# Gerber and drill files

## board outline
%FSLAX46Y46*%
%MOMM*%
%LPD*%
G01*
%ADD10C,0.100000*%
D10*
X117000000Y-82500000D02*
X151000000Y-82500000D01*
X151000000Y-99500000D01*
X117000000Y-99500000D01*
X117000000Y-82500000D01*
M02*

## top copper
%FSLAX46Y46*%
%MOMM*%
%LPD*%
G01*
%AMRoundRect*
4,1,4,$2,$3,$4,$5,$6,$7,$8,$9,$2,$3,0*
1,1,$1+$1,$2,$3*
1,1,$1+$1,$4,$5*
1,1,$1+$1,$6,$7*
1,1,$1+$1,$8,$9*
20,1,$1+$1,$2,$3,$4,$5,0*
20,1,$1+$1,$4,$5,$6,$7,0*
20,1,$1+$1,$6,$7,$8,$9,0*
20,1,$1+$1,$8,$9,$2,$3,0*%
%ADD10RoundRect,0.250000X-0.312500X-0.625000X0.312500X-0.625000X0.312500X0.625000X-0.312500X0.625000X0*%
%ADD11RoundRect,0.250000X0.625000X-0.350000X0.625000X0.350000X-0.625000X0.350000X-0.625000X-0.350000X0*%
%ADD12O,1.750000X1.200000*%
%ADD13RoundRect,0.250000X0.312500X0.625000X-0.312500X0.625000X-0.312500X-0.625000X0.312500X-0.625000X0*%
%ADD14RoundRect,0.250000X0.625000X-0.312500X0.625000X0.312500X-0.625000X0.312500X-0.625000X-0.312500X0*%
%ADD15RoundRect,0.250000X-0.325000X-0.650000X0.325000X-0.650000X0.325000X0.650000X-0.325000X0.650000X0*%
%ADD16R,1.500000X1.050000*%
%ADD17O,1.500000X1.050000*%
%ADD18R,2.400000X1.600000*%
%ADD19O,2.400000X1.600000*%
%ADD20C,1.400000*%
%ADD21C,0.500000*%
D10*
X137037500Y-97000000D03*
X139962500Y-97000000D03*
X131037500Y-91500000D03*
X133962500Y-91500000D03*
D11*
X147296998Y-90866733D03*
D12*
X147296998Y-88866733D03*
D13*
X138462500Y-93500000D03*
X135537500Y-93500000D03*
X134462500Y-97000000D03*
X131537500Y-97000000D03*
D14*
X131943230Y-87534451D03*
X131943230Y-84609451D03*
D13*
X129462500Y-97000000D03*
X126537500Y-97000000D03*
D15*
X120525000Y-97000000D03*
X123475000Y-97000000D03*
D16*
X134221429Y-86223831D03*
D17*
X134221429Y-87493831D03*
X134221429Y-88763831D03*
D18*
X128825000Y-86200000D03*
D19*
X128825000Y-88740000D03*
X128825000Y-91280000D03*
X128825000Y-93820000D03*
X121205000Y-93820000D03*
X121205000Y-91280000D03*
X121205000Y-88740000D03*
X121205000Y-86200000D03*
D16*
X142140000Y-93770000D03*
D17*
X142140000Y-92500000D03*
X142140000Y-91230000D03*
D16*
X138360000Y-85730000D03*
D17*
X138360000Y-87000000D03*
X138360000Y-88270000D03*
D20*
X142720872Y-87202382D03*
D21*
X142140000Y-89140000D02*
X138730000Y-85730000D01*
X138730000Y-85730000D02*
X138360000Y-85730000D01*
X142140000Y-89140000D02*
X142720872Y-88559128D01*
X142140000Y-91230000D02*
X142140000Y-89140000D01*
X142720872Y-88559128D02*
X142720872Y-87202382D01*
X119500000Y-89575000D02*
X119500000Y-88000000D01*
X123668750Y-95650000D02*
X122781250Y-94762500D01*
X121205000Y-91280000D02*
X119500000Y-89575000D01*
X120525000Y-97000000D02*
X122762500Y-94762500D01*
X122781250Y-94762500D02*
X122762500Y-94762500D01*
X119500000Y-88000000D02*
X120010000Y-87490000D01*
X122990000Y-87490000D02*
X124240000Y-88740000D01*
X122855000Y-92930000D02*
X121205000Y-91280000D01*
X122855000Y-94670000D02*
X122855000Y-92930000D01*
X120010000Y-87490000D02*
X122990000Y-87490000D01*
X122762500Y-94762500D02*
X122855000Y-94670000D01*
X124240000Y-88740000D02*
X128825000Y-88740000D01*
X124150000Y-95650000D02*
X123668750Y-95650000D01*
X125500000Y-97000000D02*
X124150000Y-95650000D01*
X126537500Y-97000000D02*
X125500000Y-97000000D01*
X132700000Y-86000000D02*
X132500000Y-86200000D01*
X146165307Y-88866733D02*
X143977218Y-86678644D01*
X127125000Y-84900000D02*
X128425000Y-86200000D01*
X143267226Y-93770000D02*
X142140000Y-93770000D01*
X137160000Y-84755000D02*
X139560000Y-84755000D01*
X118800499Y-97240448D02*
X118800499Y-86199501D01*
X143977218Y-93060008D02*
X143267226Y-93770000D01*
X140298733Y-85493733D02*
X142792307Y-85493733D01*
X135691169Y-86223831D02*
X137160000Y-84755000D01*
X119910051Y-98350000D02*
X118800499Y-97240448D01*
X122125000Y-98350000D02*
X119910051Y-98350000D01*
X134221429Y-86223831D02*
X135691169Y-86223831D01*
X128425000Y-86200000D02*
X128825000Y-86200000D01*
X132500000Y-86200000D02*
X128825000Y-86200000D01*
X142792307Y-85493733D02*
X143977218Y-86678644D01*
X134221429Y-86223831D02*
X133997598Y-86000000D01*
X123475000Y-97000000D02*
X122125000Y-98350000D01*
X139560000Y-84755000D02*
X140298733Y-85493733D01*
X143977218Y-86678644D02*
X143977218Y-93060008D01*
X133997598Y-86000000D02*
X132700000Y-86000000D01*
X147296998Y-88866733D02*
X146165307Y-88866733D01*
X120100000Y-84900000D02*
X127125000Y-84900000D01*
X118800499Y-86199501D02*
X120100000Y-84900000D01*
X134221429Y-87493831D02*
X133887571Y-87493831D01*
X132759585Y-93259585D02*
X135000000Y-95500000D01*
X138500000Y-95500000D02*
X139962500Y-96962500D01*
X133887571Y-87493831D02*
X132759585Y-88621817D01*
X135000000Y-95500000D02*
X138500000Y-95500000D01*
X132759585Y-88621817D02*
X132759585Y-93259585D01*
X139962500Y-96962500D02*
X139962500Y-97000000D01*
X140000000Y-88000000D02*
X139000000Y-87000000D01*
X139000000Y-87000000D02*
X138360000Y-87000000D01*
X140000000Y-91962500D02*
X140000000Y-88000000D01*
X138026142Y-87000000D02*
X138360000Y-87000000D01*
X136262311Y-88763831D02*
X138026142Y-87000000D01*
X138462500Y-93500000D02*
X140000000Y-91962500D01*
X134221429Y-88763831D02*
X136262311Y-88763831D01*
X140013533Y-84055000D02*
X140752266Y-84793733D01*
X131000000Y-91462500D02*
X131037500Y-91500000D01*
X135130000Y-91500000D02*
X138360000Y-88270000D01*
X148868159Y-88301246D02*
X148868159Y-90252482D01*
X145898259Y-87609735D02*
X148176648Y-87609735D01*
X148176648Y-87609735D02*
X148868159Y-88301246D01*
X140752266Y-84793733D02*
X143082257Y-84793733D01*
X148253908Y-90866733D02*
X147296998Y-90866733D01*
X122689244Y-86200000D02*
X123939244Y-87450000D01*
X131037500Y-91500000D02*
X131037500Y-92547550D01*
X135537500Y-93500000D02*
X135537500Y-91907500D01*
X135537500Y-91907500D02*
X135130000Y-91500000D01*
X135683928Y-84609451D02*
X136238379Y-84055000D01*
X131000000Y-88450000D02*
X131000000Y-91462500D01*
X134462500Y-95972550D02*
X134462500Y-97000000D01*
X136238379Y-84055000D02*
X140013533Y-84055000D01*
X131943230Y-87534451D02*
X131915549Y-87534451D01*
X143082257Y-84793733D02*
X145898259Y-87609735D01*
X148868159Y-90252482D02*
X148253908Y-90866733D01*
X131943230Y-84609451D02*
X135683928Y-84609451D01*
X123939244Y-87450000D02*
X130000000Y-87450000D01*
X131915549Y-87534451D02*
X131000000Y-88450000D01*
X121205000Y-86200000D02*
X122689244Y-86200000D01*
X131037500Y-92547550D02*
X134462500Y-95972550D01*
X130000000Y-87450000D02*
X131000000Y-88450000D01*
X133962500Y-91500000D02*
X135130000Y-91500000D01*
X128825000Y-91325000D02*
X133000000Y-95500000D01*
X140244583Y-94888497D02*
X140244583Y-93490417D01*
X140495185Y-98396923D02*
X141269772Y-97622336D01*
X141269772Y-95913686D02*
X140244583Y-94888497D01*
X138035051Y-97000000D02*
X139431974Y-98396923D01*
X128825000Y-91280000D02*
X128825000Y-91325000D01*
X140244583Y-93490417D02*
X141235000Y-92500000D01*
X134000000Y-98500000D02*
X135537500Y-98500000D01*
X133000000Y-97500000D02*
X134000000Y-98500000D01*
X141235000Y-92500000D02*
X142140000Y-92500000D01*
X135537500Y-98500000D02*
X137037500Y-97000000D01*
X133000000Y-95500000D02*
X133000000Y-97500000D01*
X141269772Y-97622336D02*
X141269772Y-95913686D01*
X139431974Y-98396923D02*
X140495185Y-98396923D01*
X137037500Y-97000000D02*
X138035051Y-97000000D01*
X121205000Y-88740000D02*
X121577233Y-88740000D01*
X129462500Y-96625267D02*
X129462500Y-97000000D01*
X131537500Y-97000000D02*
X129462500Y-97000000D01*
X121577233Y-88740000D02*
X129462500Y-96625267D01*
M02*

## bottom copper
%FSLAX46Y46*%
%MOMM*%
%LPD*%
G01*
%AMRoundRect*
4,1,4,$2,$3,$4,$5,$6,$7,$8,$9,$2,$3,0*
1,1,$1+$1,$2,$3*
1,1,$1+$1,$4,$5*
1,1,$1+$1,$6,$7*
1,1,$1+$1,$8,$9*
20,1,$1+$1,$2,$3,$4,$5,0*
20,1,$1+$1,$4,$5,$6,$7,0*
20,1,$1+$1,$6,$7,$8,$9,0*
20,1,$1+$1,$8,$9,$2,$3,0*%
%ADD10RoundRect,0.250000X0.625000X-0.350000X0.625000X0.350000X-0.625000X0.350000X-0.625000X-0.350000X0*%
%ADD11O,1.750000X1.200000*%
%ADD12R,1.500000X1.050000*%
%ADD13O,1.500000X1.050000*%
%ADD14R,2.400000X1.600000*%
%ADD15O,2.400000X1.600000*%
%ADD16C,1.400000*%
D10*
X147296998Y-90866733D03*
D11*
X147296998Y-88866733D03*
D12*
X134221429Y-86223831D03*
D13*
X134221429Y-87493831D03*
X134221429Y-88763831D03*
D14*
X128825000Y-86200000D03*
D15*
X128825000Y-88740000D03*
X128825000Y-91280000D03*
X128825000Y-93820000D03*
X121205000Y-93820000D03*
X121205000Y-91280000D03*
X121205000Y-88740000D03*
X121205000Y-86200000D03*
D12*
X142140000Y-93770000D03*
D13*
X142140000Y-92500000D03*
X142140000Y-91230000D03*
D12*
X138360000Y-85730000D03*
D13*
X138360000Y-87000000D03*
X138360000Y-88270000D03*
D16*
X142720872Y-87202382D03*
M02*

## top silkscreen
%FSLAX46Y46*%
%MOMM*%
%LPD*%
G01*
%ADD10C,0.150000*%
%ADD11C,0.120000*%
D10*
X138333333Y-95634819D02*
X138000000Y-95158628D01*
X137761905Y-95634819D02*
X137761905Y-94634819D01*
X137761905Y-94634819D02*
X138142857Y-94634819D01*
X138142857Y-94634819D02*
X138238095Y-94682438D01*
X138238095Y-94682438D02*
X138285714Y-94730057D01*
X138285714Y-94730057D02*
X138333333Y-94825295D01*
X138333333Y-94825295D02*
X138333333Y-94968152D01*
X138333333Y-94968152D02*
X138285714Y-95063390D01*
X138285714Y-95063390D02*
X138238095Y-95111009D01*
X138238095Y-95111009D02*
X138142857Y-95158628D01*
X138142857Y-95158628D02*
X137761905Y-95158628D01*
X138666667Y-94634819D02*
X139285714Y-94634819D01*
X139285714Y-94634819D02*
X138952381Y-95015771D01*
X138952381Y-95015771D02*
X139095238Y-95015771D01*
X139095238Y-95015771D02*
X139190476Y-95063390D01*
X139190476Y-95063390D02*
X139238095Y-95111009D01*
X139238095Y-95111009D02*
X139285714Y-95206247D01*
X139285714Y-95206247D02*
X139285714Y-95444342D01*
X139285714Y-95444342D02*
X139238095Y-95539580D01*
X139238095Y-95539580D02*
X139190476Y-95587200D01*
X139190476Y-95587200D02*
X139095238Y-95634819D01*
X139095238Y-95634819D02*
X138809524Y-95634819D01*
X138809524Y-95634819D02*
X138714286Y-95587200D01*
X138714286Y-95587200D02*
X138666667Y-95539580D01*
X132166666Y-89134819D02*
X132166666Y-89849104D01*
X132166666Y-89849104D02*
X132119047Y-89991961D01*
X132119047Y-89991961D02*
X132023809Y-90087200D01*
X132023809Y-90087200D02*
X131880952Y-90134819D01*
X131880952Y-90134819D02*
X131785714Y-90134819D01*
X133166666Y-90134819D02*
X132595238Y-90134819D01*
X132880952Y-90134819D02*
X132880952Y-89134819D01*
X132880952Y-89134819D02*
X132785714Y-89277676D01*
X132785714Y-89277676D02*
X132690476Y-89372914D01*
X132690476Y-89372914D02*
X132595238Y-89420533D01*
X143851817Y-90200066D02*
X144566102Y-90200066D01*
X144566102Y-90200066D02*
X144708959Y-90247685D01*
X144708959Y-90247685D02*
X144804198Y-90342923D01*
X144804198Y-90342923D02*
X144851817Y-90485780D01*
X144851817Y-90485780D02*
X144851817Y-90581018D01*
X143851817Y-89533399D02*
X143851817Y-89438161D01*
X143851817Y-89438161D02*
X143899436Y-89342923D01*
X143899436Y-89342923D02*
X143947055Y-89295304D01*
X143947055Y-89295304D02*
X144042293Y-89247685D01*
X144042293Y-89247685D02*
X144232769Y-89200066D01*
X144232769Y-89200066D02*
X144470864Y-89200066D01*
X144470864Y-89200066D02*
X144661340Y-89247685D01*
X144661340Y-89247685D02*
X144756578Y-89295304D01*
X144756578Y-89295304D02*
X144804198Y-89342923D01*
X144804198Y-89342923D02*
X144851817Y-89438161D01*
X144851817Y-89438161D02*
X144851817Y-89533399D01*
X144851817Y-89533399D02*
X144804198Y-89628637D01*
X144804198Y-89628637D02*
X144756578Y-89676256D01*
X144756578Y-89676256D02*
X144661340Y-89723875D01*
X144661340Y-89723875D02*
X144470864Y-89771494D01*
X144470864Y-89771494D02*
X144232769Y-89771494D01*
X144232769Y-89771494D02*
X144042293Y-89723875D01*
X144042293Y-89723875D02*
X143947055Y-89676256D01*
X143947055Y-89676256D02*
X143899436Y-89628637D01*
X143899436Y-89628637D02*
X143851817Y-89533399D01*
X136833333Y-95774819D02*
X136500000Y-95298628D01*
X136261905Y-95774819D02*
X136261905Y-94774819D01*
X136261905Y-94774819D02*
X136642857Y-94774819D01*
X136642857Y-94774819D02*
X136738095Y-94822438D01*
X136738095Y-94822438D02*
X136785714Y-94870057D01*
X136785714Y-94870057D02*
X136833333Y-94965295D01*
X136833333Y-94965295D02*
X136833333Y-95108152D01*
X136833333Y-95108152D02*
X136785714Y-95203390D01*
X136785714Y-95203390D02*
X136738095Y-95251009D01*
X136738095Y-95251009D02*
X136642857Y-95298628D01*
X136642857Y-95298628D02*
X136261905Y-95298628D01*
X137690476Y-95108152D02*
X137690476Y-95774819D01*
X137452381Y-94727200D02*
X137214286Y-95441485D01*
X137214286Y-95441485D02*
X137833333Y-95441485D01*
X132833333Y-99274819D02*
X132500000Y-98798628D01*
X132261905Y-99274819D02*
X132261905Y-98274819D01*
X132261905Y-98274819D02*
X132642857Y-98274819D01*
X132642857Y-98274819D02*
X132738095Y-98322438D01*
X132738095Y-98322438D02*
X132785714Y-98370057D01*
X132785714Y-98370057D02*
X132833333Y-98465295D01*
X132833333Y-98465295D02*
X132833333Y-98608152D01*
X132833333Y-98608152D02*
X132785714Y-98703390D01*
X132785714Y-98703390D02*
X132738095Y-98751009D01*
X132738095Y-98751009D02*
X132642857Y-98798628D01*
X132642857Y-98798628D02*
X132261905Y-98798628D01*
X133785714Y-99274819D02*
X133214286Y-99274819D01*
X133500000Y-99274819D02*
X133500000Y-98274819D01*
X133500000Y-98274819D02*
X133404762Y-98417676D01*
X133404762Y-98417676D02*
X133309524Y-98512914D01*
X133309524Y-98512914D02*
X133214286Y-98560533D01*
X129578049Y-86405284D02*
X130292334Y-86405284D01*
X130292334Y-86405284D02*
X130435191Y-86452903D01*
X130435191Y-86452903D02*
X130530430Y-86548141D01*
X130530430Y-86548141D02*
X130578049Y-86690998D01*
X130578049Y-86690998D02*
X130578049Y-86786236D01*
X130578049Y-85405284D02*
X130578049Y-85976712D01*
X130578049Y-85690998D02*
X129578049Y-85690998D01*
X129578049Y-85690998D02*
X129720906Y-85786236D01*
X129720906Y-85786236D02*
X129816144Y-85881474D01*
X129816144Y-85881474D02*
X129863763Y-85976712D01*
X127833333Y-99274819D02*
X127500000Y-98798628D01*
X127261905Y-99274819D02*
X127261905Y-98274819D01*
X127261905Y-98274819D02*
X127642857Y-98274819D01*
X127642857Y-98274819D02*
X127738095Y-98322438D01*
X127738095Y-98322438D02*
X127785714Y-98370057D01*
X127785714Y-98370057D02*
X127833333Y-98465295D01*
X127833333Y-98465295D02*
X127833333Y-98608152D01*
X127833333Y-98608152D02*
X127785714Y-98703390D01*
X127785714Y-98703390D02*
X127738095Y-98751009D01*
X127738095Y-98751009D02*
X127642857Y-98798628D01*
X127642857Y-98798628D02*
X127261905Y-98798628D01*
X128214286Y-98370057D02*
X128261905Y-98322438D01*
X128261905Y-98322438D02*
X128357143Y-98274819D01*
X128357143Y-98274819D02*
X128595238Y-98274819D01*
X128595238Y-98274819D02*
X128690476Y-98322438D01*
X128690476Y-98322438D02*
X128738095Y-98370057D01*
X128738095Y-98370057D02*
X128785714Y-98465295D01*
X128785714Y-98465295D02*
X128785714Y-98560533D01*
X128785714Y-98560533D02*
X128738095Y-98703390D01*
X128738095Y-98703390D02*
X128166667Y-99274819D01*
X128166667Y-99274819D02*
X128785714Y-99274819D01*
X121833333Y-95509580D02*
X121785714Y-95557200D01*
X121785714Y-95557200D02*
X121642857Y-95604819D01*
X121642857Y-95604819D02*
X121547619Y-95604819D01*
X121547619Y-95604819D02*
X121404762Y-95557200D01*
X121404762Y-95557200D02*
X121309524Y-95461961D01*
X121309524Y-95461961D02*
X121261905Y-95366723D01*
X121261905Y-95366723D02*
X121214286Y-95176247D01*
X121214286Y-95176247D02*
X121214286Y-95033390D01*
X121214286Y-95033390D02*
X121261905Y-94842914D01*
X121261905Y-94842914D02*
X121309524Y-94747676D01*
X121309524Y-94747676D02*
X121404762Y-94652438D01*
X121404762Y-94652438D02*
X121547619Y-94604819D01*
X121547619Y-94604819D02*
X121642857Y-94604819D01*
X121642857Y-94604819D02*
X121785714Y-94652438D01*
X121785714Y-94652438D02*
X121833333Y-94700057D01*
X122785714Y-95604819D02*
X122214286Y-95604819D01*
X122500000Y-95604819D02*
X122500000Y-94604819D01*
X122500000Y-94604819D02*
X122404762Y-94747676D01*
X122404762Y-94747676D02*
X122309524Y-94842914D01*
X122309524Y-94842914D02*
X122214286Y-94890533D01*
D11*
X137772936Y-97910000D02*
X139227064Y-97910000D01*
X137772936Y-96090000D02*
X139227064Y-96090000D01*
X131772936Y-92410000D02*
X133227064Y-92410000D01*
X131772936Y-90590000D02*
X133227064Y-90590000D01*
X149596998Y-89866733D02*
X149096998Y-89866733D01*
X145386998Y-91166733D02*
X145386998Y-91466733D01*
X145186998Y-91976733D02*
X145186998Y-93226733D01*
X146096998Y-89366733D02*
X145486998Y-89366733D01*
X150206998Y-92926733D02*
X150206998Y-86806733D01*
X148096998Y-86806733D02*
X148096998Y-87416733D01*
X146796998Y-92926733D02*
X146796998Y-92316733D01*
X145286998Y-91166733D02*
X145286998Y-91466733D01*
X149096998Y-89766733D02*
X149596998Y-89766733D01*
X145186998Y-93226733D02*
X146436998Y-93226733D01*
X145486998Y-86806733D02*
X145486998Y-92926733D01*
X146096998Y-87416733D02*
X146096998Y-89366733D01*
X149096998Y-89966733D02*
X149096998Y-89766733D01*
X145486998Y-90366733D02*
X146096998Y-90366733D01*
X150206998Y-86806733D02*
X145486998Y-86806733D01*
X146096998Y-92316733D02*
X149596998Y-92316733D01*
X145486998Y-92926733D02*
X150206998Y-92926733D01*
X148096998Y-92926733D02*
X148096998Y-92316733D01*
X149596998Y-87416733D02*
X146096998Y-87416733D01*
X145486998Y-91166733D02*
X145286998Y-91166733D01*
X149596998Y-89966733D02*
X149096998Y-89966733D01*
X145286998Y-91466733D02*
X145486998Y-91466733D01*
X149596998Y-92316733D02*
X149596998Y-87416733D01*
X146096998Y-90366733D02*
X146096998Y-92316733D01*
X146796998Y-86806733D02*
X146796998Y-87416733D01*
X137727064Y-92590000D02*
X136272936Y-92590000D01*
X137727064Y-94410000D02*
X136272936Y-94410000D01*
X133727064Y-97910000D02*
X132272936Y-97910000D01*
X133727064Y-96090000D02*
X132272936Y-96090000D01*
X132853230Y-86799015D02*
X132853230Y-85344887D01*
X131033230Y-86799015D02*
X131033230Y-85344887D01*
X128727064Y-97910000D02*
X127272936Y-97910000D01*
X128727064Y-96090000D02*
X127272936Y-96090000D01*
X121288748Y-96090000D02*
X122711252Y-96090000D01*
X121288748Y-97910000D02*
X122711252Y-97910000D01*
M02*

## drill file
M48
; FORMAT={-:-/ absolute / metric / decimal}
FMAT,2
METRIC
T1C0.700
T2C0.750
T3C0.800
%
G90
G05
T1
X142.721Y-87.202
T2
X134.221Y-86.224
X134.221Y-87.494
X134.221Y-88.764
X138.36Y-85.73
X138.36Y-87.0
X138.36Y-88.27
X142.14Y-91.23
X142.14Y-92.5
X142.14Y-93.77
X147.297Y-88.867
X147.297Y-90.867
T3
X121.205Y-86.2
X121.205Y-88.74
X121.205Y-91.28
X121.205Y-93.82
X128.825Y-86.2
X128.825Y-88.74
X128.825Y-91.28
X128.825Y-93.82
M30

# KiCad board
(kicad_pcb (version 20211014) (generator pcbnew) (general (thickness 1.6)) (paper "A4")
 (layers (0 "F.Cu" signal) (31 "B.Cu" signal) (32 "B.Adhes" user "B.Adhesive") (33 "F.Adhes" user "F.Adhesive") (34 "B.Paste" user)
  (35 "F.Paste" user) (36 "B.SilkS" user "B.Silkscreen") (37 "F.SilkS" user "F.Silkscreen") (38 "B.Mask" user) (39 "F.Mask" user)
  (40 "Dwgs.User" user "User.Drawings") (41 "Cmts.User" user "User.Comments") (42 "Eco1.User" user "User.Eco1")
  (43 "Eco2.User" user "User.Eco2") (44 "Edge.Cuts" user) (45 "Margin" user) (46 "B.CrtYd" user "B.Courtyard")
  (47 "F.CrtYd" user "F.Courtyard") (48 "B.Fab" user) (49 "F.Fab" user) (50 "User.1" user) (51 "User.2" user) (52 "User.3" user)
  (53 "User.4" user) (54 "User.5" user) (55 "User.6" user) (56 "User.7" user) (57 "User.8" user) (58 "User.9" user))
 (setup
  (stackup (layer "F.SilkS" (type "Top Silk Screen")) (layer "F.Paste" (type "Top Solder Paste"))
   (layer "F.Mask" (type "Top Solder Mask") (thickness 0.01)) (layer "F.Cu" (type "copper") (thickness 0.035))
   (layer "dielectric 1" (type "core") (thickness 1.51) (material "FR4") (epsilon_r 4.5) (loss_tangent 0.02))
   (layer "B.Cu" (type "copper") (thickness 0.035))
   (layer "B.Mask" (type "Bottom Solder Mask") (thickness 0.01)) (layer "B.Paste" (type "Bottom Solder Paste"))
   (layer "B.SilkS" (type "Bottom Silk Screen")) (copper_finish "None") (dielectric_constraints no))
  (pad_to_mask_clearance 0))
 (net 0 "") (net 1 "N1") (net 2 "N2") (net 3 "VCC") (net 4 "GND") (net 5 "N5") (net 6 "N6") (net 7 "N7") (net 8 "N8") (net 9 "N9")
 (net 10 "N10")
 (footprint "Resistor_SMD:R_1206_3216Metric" (layer "F.Cu") (at 138.5 97)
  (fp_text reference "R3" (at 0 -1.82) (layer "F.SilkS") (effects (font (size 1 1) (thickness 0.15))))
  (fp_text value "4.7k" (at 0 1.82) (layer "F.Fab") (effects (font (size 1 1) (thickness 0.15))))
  (fp_line (start -0.727064 0.91) (end 0.727064 0.91) (layer "F.SilkS") (width 0.12))
  (fp_line (start -0.727064 -0.91) (end 0.727064 -0.91) (layer "F.SilkS") (width 0.12))
  (pad "1" smd roundrect (at -1.4625 0) (size 1.125 1.75) (layers "F.Cu" "F.Paste" "F.Mask") (roundrect_rratio 0.2222222222) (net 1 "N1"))
  (pad "2" smd roundrect (at 1.4625 0) (size 1.125 1.75) (layers "F.Cu" "F.Paste" "F.Mask") (roundrect_rratio 0.2222222222) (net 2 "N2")))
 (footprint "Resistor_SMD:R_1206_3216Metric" (layer "F.Cu") (at 132.5 91.5)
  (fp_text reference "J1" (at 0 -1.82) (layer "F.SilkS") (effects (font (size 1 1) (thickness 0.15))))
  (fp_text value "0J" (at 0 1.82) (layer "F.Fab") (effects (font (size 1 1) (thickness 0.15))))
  (fp_line (start -0.727064 0.91) (end 0.727064 0.91) (layer "F.SilkS") (width 0.12))
  (fp_line (start -0.727064 -0.91) (end 0.727064 -0.91) (layer "F.SilkS") (width 0.12))
  (pad "1" smd roundrect (at -1.4625 0) (size 1.125 1.75) (layers "F.Cu" "F.Paste" "F.Mask") (roundrect_rratio 0.2222222222) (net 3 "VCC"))
  (pad "2" smd roundrect (at 1.4625 0) (size 1.125 1.75) (layers "F.Cu" "F.Paste" "F.Mask") (roundrect_rratio 0.2222222222) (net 3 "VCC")))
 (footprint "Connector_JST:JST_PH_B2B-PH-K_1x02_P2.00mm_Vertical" (layer "F.Cu") (at 147.296998 90.866733 90)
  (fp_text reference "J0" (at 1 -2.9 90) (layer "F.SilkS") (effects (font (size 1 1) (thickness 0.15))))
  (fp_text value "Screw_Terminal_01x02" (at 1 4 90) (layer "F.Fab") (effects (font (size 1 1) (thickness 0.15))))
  (fp_line (start 1 2.3) (end 1 1.8) (layer "F.SilkS") (width 0.12))
  (fp_line (start -0.3 -1.91) (end -0.6 -1.91) (layer "F.SilkS") (width 0.12))
  (fp_line (start -1.11 -2.11) (end -2.36 -2.11) (layer "F.SilkS") (width 0.12))
  (fp_line (start 1.5 -1.2) (end 1.5 -1.81) (layer "F.SilkS") (width 0.12))
  (fp_line (start -2.06 2.91) (end 4.06 2.91) (layer "F.SilkS") (width 0.12))
  (fp_line (start 4.06 0.8) (end 3.45 0.8) (layer "F.SilkS") (width 0.12))
  (fp_line (start -2.06 -0.5) (end -1.45 -0.5) (layer "F.SilkS") (width 0.12))
  (fp_line (start -0.3 -2.01) (end -0.6 -2.01) (layer "F.SilkS") (width 0.12))
  (fp_line (start 1.1 1.8) (end 1.1 2.3) (layer "F.SilkS") (width 0.12))
  (fp_line (start -2.36 -2.11) (end -2.36 -0.86) (layer "F.SilkS") (width 0.12))
  (fp_line (start 4.06 -1.81) (end -2.06 -1.81) (layer "F.SilkS") (width 0.12))
  (fp_line (start 3.45 -1.2) (end 1.5 -1.2) (layer "F.SilkS") (width 0.12))
  (fp_line (start 0.9 1.8) (end 1.1 1.8) (layer "F.SilkS") (width 0.12))
  (fp_line (start 0.5 -1.81) (end 0.5 -1.2) (layer "F.SilkS") (width 0.12))
  (fp_line (start 4.06 2.91) (end 4.06 -1.81) (layer "F.SilkS") (width 0.12))
  (fp_line (start -1.45 -1.2) (end -1.45 2.3) (layer "F.SilkS") (width 0.12))
  (fp_line (start -2.06 -1.81) (end -2.06 2.91) (layer "F.SilkS") (width 0.12))
  (fp_line (start -2.06 0.8) (end -1.45 0.8) (layer "F.SilkS") (width 0.12))
  (fp_line (start 3.45 2.3) (end 3.45 -1.2) (layer "F.SilkS") (width 0.12))
  (fp_line (start -0.3 -1.81) (end -0.3 -2.01) (layer "F.SilkS") (width 0.12))
  (fp_line (start 0.9 2.3) (end 0.9 1.8) (layer "F.SilkS") (width 0.12))
  (fp_line (start -0.6 -2.01) (end -0.6 -1.81) (layer "F.SilkS") (width 0.12))
  (fp_line (start -1.45 2.3) (end 3.45 2.3) (layer "F.SilkS") (width 0.12))
  (fp_line (start 0.5 -1.2) (end -1.45 -1.2) (layer "F.SilkS") (width 0.12))
  (fp_line (start 4.06 -0.5) (end 3.45 -0.5) (layer "F.SilkS") (width 0.12))
  (pad "1" thru_hole roundrect (at 0 0 90) (size 1.2 1.75) (drill 0.75) (layers *.Cu *.Mask) (roundrect_rratio 0.2083333333) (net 3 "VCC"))
  (pad "2" thru_hole oval (at 2 0 90) (size 1.2 1.75) (drill 0.75) (layers *.Cu *.Mask) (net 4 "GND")))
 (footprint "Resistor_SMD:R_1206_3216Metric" (layer "F.Cu") (at 137 93.5 180)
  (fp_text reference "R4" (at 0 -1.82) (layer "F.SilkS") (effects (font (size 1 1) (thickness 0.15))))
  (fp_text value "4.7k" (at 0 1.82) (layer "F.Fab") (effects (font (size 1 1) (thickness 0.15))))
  (fp_line (start -0.727064 0.91) (end 0.727064 0.91) (layer "F.SilkS") (width 0.12))
  (fp_line (start -0.727064 -0.91) (end 0.727064 -0.91) (layer "F.SilkS") (width 0.12))
  (pad "1" smd roundrect (at -1.4625 0 180) (size 1.125 1.75) (layers "F.Cu" "F.Paste" "F.Mask") (roundrect_rratio 0.2222222222)
   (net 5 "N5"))
  (pad "2" smd roundrect (at 1.4625 0 180) (size 1.125 1.75) (layers "F.Cu" "F.Paste" "F.Mask") (roundrect_rratio 0.2222222222)
   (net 3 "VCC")))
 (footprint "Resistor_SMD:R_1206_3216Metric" (layer "F.Cu") (at 133 97 180)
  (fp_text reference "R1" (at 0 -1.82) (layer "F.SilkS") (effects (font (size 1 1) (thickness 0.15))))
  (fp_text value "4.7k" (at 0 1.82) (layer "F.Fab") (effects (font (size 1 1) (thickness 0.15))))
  (fp_line (start -0.727064 -0.91) (end 0.727064 -0.91) (layer "F.SilkS") (width 0.12))
  (fp_line (start -0.727064 0.91) (end 0.727064 0.91) (layer "F.SilkS") (width 0.12))
  (pad "1" smd roundrect (at -1.4625 0 180) (size 1.125 1.75) (layers "F.Cu" "F.Paste" "F.Mask") (roundrect_rratio 0.2222222222)
   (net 3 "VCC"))
  (pad "2" smd roundrect (at 1.4625 0 180) (size 1.125 1.75) (layers "F.Cu" "F.Paste" "F.Mask") (roundrect_rratio 0.2222222222) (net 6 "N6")))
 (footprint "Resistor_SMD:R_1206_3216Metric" (layer "F.Cu") (at 131.94323 86.071951 90)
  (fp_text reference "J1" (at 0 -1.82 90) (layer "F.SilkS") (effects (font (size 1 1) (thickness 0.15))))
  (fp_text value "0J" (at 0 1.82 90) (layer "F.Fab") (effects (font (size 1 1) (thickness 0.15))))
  (fp_line (start -0.727064 0.91) (end 0.727064 0.91) (layer "F.SilkS") (width 0.12))
  (fp_line (start -0.727064 -0.91) (end 0.727064 -0.91) (layer "F.SilkS") (width 0.12))
  (pad "1" smd roundrect (at -1.4625 0 90) (size 1.125 1.75) (layers "F.Cu" "F.Paste" "F.Mask") (roundrect_rratio 0.2222222222)
   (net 3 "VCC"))
  (pad "2" smd roundrect (at 1.4625 0 90) (size 1.125 1.75) (layers "F.Cu" "F.Paste" "F.Mask") (roundrect_rratio 0.2222222222) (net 3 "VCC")))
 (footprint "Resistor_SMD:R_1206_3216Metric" (layer "F.Cu") (at 128 97 180)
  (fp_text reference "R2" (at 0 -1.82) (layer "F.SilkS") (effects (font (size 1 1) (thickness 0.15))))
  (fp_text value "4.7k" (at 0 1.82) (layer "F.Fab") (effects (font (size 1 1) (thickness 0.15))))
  (fp_line (start -0.727064 -0.91) (end 0.727064 -0.91) (layer "F.SilkS") (width 0.12))
  (fp_line (start -0.727064 0.91) (end 0.727064 0.91) (layer "F.SilkS") (width 0.12))
  (pad "1" smd roundrect (at -1.4625 0 180) (size 1.125 1.75) (layers "F.Cu" "F.Paste" "F.Mask") (roundrect_rratio 0.2222222222)
   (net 6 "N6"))
  (pad "2" smd roundrect (at 1.4625 0 180) (size 1.125 1.75) (layers "F.Cu" "F.Paste" "F.Mask") (roundrect_rratio 0.2222222222) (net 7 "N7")))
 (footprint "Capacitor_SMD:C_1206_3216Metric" (layer "F.Cu") (at 122 97)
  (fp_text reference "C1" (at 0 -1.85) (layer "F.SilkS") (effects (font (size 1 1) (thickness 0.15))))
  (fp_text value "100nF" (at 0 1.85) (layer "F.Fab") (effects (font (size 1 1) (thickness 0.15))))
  (fp_line (start -0.711252 -0.91) (end 0.711252 -0.91) (layer "F.SilkS") (width 0.12))
  (fp_line (start -0.711252 0.91) (end 0.711252 0.91) (layer "F.SilkS") (width 0.12))
  (pad "1" smd roundrect (at -1.475 0) (size 1.15 1.8) (layers "F.Cu" "F.Paste" "F.Mask") (roundrect_rratio 0.2173913043) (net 7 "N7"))
  (pad "2" smd roundrect (at 1.475 0) (size 1.15 1.8) (layers "F.Cu" "F.Paste" "F.Mask") (roundrect_rratio 0.2173913043) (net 4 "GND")))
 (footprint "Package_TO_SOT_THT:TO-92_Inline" (layer "B.Cu") (at 134.221429 86.223831 -90)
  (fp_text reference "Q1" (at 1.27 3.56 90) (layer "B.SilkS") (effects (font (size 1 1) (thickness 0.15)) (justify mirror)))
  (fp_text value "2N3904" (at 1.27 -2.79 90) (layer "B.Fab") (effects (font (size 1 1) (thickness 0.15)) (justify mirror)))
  (pad "1" thru_hole rect (at 0 0 270) (size 1.05 1.5) (drill 0.75) (layers *.Cu *.Mask) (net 4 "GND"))
  (pad "2" thru_hole oval (at 1.27 0 270) (size 1.05 1.5) (drill 0.75) (layers *.Cu *.Mask) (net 2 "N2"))
  (pad "3" thru_hole oval (at 2.54 0 270) (size 1.05 1.5) (drill 0.75) (layers *.Cu *.Mask) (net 5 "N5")))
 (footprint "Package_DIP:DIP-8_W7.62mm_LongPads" (layer "B.Cu") (at 128.825 86.2 180)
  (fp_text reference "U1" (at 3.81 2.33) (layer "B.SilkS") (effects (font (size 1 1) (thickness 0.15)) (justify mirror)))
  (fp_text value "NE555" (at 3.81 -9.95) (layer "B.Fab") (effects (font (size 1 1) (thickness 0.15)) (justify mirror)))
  (pad "1" thru_hole rect (at 0 0 180) (size 2.4 1.6) (drill 0.8) (layers *.Cu *.Mask) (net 4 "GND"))
  (pad "2" thru_hole oval (at 0 -2.54 180) (size 2.4 1.6) (drill 0.8) (layers *.Cu *.Mask) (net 7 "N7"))
  (pad "3" thru_hole oval (at 0 -5.08 180) (size 2.4 1.6) (drill 0.8) (layers *.Cu *.Mask) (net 1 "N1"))
  (pad "4" thru_hole oval (at 0 -7.62 180) (size 2.4 1.6) (drill 0.8) (layers *.Cu *.Mask) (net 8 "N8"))
  (pad "5" thru_hole oval (at 7.62 -7.62 180) (size 2.4 1.6) (drill 0.8) (layers *.Cu *.Mask) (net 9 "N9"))
  (pad "6" thru_hole oval (at 7.62 -5.08 180) (size 2.4 1.6) (drill 0.8) (layers *.Cu *.Mask) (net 7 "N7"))
  (pad "7" thru_hole oval (at 7.62 -2.54 180) (size 2.4 1.6) (drill 0.8) (layers *.Cu *.Mask) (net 6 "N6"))
  (pad "8" thru_hole oval (at 7.62 0 180) (size 2.4 1.6) (drill 0.8) (layers *.Cu *.Mask) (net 3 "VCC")))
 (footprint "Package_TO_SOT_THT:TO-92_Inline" (layer "B.Cu") (at 142.14 93.77 90)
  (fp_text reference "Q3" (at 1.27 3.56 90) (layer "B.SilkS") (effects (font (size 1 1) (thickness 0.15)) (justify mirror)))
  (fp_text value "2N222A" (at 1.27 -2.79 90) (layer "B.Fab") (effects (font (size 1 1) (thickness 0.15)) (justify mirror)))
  (pad "1" thru_hole rect (at 0 0 90) (size 1.05 1.5) (drill 0.75) (layers *.Cu *.Mask) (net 4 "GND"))
  (pad "2" thru_hole oval (at 1.27 0 90) (size 1.05 1.5) (drill 0.75) (layers *.Cu *.Mask) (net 1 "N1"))
  (pad "3" thru_hole oval (at 2.54 0 90) (size 1.05 1.5) (drill 0.75) (layers *.Cu *.Mask) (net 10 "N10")))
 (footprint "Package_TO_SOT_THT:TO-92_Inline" (layer "B.Cu") (at 138.36 85.73 -90)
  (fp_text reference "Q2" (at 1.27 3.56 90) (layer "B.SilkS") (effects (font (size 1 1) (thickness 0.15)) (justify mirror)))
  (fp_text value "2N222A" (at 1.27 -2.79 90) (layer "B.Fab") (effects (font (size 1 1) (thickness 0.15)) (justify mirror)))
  (pad "1" thru_hole rect (at 0 0 270) (size 1.05 1.5) (drill 0.75) (layers *.Cu *.Mask) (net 10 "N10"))
  (pad "2" thru_hole oval (at 1.27 0 270) (size 1.05 1.5) (drill 0.75) (layers *.Cu *.Mask) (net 5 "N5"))
  (pad "3" thru_hole oval (at 2.54 0 270) (size 1.05 1.5) (drill 0.75) (layers *.Cu *.Mask) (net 3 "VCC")))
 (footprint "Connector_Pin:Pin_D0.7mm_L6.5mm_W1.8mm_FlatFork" (layer "B.Cu") (at 142.720872 87.202382 180)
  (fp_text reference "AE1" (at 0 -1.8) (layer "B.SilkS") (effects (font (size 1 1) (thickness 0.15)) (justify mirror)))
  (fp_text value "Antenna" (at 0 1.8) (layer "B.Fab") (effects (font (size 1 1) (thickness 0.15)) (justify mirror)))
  (pad "1" thru_hole circle (at 0 0 180) (size 1.4 1.4) (drill 0.7) (layers *.Cu *.Mask) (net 10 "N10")))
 (gr_rect (start 117 82.5) (end 151 99.5) (layer "Edge.Cuts") (width 0.1) (fill none))
 (segment (start 142.14 89.14) (end 138.73 85.73) (width 0.5) (layer "F.Cu") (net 10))
 (segment (start 138.73 85.73) (end 138.36 85.73) (width 0.5) (layer "F.Cu") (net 10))
 (segment (start 142.14 89.14) (end 142.720872 88.559128) (width 0.5) (layer "F.Cu") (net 10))
 (segment (start 142.14 91.23) (end 142.14 89.14) (width 0.5) (layer "F.Cu") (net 10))
 (segment (start 142.720872 88.559128) (end 142.720872 87.202382) (width 0.5) (layer "F.Cu") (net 10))
 (segment (start 119.5 89.575) (end 119.5 88) (width 0.5) (layer "F.Cu") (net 7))
 (segment (start 123.66875 95.65) (end 122.78125 94.7625) (width 0.5) (layer "F.Cu") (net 7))
 (segment (start 121.205 91.28) (end 119.5 89.575) (width 0.5) (layer "F.Cu") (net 7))
 (segment (start 120.525 97) (end 122.7625 94.7625) (width 0.5) (layer "F.Cu") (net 7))
 (segment (start 122.78125 94.7625) (end 122.7625 94.7625) (width 0.5) (layer "F.Cu") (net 7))
 (segment (start 119.5 88) (end 120.01 87.49) (width 0.5) (layer "F.Cu") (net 7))
 (segment (start 122.99 87.49) (end 124.24 88.74) (width 0.5) (layer "F.Cu") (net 7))
 (segment (start 122.855 92.93) (end 121.205 91.28) (width 0.5) (layer "F.Cu") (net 7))
 (segment (start 122.855 94.67) (end 122.855 92.93) (width 0.5) (layer "F.Cu") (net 7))
 (segment (start 120.01 87.49) (end 122.99 87.49) (width 0.5) (layer "F.Cu") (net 7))
 (segment (start 122.7625 94.7625) (end 122.855 94.67) (width 0.5) (layer "F.Cu") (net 7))
 (segment (start 124.24 88.74) (end 128.825 88.74) (width 0.5) (layer "F.Cu") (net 7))
 (segment (start 124.15 95.65) (end 123.66875 95.65) (width 0.5) (layer "F.Cu") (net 7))
 (segment (start 125.5 97) (end 124.15 95.65) (width 0.5) (layer "F.Cu") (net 7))
 (segment (start 126.5375 97) (end 125.5 97) (width 0.5) (layer "F.Cu") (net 7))
 (segment (start 132.7 86) (end 132.5 86.2) (width 0.5) (layer "F.Cu") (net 4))
 (segment (start 146.165307 88.866733) (end 143.977218 86.678644) (width 0.5) (layer "F.Cu") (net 4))
 (segment (start 127.125 84.9) (end 128.425 86.2) (width 0.5) (layer "F.Cu") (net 4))
 (segment (start 143.267226 93.77) (end 142.14 93.77) (width 0.5) (layer "F.Cu") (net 4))
 (segment (start 137.16 84.755) (end 139.56 84.755) (width 0.5) (layer "F.Cu") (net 4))
 (segment (start 118.800499 97.240448) (end 118.800499 86.199501) (width 0.5) (layer "F.Cu") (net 4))
 (segment (start 143.977218 93.060008) (end 143.267226 93.77) (width 0.5) (layer "F.Cu") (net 4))
 (segment (start 140.298733 85.493733) (end 142.792307 85.493733) (width 0.5) (layer "F.Cu") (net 4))
 (segment (start 135.691169 86.223831) (end 137.16 84.755) (width 0.5) (layer "F.Cu") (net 4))
 (segment (start 119.910051 98.35) (end 118.800499 97.240448) (width 0.5) (layer "F.Cu") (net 4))
 (segment (start 122.125 98.35) (end 119.910051 98.35) (width 0.5) (layer "F.Cu") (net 4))
 (segment (start 134.221429 86.223831) (end 135.691169 86.223831) (width 0.5) (layer "F.Cu") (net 4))
 (segment (start 128.425 86.2) (end 128.825 86.2) (width 0.5) (layer "F.Cu") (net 4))
 (segment (start 132.5 86.2) (end 128.825 86.2) (width 0.5) (layer "F.Cu") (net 4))
 (segment (start 142.792307 85.493733) (end 143.977218 86.678644) (width 0.5) (layer "F.Cu") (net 4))
 (segment (start 134.221429 86.223831) (end 133.997598 86) (width 0.5) (layer "F.Cu") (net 4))
 (segment (start 123.475 97) (end 122.125 98.35) (width 0.5) (layer "F.Cu") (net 4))
 (segment (start 139.56 84.755) (end 140.298733 85.493733) (width 0.5) (layer "F.Cu") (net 4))
 (segment (start 143.977218 86.678644) (end 143.977218 93.060008) (width 0.5) (layer "F.Cu") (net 4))
 (segment (start 133.997598 86) (end 132.7 86) (width 0.5) (layer "F.Cu") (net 4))
 (segment (start 147.296998 88.866733) (end 146.165307 88.866733) (width 0.5) (layer "F.Cu") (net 4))
 (segment (start 120.1 84.9) (end 127.125 84.9) (width 0.5) (layer "F.Cu") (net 4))
 (segment (start 118.800499 86.199501) (end 120.1 84.9) (width 0.5) (layer "F.Cu") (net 4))
 (segment (start 134.221429 87.493831) (end 133.887571 87.493831) (width 0.5) (layer "F.Cu") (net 2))
 (segment (start 132.759585 93.259585) (end 135 95.5) (width 0.5) (layer "F.Cu") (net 2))
 (segment (start 138.5 95.5) (end 139.9625 96.9625) (width 0.5) (layer "F.Cu") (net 2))
 (segment (start 133.887571 87.493831) (end 132.759585 88.621817) (width 0.5) (layer "F.Cu") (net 2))
 (segment (start 135 95.5) (end 138.5 95.5) (width 0.5) (layer "F.Cu") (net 2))
 (segment (start 132.759585 88.621817) (end 132.759585 93.259585) (width 0.5) (layer "F.Cu") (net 2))
 (segment (start 139.9625 96.9625) (end 139.9625 97) (width 0.5) (layer "F.Cu") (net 2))
 (segment (start 140 88) (end 139 87) (width 0.5) (layer "F.Cu") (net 5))
 (segment (start 139 87) (end 138.36 87) (width 0.5) (layer "F.Cu") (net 5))
 (segment (start 140 91.9625) (end 140 88) (width 0.5) (layer "F.Cu") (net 5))
 (segment (start 138.026142 87) (end 138.36 87) (width 0.5) (layer "F.Cu") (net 5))
 (segment (start 136.262311 88.763831) (end 138.026142 87) (width 0.5) (layer "F.Cu") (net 5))
 (segment (start 138.4625 93.5) (end 140 91.9625) (width 0.5) (layer "F.Cu") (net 5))
 (segment (start 134.221429 88.763831) (end 136.262311 88.763831) (width 0.5) (layer "F.Cu") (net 5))
 (segment (start 140.013533 84.055) (end 140.752266 84.793733) (width 0.5) (layer "F.Cu") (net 3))
 (segment (start 131 91.4625) (end 131.0375 91.5) (width 0.5) (layer "F.Cu") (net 3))
 (segment (start 135.13 91.5) (end 138.36 88.27) (width 0.5) (layer "F.Cu") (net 3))
 (segment (start 148.868159 88.301246) (end 148.868159 90.252482) (width 0.5) (layer "F.Cu") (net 3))
 (segment (start 145.898259 87.609735) (end 148.176648 87.609735) (width 0.5) (layer "F.Cu") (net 3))
 (segment (start 148.176648 87.609735) (end 148.868159 88.301246) (width 0.5) (layer "F.Cu") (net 3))
 (segment (start 140.752266 84.793733) (end 143.082257 84.793733) (width 0.5) (layer "F.Cu") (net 3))
 (segment (start 148.253908 90.866733) (end 147.296998 90.866733) (width 0.5) (layer "F.Cu") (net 3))
 (segment (start 122.689244 86.2) (end 123.939244 87.45) (width 0.5) (layer "F.Cu") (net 3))
 (segment (start 131.0375 91.5) (end 131.0375 92.54755) (width 0.5) (layer "F.Cu") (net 3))
 (segment (start 135.5375 93.5) (end 135.5375 91.9075) (width 0.5) (layer "F.Cu") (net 3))
 (segment (start 135.5375 91.9075) (end 135.13 91.5) (width 0.5) (layer "F.Cu") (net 3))
 (segment (start 135.683928 84.609451) (end 136.238379 84.055) (width 0.5) (layer "F.Cu") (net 3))
 (segment (start 131 88.45) (end 131 91.4625) (width 0.5) (layer "F.Cu") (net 3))
 (segment (start 134.4625 95.97255) (end 134.4625 97) (width 0.5) (layer "F.Cu") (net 3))
 (segment (start 136.238379 84.055) (end 140.013533 84.055) (width 0.5) (layer "F.Cu") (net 3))
 (segment (start 131.94323 87.534451) (end 131.915549 87.534451) (width 0.5) (layer "F.Cu") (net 3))
 (segment (start 143.082257 84.793733) (end 145.898259 87.609735) (width 0.5) (layer "F.Cu") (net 3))
 (segment (start 148.868159 90.252482) (end 148.253908 90.866733) (width 0.5) (layer "F.Cu") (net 3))
 (segment (start 131.94323 84.609451) (end 135.683928 84.609451) (width 0.5) (layer "F.Cu") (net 3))
 (segment (start 123.939244 87.45) (end 130 87.45) (width 0.5) (layer "F.Cu") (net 3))
 (segment (start 131.915549 87.534451) (end 131 88.45) (width 0.5) (layer "F.Cu") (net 3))
 (segment (start 121.205 86.2) (end 122.689244 86.2) (width 0.5) (layer "F.Cu") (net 3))
 (segment (start 131.0375 92.54755) (end 134.4625 95.97255) (width 0.5) (layer "F.Cu") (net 3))
 (segment (start 130 87.45) (end 131 88.45) (width 0.5) (layer "F.Cu") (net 3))
 (segment (start 133.9625 91.5) (end 135.13 91.5) (width 0.5) (layer "F.Cu") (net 3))
 (segment (start 128.825 91.325) (end 133 95.5) (width 0.5) (layer "F.Cu") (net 1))
 (segment (start 140.244583 94.888497) (end 140.244583 93.490417) (width 0.5) (layer "F.Cu") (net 1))
 (segment (start 140.495185 98.396923) (end 141.269772 97.622336) (width 0.5) (layer "F.Cu") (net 1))
 (segment (start 141.269772 95.913686) (end 140.244583 94.888497) (width 0.5) (layer "F.Cu") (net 1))
 (segment (start 138.035051 97) (end 139.431974 98.396923) (width 0.5) (layer "F.Cu") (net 1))
 (segment (start 128.825 91.28) (end 128.825 91.325) (width 0.5) (layer "F.Cu") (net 1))
 (segment (start 140.244583 93.490417) (end 141.235 92.5) (width 0.5) (layer "F.Cu") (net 1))
 (segment (start 134 98.5) (end 135.5375 98.5) (width 0.5) (layer "F.Cu") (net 1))
 (segment (start 133 97.5) (end 134 98.5) (width 0.5) (layer "F.Cu") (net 1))
 (segment (start 141.235 92.5) (end 142.14 92.5) (width 0.5) (layer "F.Cu") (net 1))
 (segment (start 135.5375 98.5) (end 137.0375 97) (width 0.5) (layer "F.Cu") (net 1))
 (segment (start 133 95.5) (end 133 97.5) (width 0.5) (layer "F.Cu") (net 1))
 (segment (start 141.269772 97.622336) (end 141.269772 95.913686) (width 0.5) (layer "F.Cu") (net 1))
 (segment (start 139.431974 98.396923) (end 140.495185 98.396923) (width 0.5) (layer "F.Cu") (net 1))
 (segment (start 137.0375 97) (end 138.035051 97) (width 0.5) (layer "F.Cu") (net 1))
 (segment (start 121.205 88.74) (end 121.577233 88.74) (width 0.5) (layer "F.Cu") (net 6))
 (segment (start 129.4625 96.625267) (end 129.4625 97) (width 0.5) (layer "F.Cu") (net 6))
 (segment (start 131.5375 97) (end 129.4625 97) (width 0.5) (layer "F.Cu") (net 6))
 (segment (start 121.577233 88.74) (end 129.4625 96.625267) (width 0.5) (layer "F.Cu") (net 6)))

